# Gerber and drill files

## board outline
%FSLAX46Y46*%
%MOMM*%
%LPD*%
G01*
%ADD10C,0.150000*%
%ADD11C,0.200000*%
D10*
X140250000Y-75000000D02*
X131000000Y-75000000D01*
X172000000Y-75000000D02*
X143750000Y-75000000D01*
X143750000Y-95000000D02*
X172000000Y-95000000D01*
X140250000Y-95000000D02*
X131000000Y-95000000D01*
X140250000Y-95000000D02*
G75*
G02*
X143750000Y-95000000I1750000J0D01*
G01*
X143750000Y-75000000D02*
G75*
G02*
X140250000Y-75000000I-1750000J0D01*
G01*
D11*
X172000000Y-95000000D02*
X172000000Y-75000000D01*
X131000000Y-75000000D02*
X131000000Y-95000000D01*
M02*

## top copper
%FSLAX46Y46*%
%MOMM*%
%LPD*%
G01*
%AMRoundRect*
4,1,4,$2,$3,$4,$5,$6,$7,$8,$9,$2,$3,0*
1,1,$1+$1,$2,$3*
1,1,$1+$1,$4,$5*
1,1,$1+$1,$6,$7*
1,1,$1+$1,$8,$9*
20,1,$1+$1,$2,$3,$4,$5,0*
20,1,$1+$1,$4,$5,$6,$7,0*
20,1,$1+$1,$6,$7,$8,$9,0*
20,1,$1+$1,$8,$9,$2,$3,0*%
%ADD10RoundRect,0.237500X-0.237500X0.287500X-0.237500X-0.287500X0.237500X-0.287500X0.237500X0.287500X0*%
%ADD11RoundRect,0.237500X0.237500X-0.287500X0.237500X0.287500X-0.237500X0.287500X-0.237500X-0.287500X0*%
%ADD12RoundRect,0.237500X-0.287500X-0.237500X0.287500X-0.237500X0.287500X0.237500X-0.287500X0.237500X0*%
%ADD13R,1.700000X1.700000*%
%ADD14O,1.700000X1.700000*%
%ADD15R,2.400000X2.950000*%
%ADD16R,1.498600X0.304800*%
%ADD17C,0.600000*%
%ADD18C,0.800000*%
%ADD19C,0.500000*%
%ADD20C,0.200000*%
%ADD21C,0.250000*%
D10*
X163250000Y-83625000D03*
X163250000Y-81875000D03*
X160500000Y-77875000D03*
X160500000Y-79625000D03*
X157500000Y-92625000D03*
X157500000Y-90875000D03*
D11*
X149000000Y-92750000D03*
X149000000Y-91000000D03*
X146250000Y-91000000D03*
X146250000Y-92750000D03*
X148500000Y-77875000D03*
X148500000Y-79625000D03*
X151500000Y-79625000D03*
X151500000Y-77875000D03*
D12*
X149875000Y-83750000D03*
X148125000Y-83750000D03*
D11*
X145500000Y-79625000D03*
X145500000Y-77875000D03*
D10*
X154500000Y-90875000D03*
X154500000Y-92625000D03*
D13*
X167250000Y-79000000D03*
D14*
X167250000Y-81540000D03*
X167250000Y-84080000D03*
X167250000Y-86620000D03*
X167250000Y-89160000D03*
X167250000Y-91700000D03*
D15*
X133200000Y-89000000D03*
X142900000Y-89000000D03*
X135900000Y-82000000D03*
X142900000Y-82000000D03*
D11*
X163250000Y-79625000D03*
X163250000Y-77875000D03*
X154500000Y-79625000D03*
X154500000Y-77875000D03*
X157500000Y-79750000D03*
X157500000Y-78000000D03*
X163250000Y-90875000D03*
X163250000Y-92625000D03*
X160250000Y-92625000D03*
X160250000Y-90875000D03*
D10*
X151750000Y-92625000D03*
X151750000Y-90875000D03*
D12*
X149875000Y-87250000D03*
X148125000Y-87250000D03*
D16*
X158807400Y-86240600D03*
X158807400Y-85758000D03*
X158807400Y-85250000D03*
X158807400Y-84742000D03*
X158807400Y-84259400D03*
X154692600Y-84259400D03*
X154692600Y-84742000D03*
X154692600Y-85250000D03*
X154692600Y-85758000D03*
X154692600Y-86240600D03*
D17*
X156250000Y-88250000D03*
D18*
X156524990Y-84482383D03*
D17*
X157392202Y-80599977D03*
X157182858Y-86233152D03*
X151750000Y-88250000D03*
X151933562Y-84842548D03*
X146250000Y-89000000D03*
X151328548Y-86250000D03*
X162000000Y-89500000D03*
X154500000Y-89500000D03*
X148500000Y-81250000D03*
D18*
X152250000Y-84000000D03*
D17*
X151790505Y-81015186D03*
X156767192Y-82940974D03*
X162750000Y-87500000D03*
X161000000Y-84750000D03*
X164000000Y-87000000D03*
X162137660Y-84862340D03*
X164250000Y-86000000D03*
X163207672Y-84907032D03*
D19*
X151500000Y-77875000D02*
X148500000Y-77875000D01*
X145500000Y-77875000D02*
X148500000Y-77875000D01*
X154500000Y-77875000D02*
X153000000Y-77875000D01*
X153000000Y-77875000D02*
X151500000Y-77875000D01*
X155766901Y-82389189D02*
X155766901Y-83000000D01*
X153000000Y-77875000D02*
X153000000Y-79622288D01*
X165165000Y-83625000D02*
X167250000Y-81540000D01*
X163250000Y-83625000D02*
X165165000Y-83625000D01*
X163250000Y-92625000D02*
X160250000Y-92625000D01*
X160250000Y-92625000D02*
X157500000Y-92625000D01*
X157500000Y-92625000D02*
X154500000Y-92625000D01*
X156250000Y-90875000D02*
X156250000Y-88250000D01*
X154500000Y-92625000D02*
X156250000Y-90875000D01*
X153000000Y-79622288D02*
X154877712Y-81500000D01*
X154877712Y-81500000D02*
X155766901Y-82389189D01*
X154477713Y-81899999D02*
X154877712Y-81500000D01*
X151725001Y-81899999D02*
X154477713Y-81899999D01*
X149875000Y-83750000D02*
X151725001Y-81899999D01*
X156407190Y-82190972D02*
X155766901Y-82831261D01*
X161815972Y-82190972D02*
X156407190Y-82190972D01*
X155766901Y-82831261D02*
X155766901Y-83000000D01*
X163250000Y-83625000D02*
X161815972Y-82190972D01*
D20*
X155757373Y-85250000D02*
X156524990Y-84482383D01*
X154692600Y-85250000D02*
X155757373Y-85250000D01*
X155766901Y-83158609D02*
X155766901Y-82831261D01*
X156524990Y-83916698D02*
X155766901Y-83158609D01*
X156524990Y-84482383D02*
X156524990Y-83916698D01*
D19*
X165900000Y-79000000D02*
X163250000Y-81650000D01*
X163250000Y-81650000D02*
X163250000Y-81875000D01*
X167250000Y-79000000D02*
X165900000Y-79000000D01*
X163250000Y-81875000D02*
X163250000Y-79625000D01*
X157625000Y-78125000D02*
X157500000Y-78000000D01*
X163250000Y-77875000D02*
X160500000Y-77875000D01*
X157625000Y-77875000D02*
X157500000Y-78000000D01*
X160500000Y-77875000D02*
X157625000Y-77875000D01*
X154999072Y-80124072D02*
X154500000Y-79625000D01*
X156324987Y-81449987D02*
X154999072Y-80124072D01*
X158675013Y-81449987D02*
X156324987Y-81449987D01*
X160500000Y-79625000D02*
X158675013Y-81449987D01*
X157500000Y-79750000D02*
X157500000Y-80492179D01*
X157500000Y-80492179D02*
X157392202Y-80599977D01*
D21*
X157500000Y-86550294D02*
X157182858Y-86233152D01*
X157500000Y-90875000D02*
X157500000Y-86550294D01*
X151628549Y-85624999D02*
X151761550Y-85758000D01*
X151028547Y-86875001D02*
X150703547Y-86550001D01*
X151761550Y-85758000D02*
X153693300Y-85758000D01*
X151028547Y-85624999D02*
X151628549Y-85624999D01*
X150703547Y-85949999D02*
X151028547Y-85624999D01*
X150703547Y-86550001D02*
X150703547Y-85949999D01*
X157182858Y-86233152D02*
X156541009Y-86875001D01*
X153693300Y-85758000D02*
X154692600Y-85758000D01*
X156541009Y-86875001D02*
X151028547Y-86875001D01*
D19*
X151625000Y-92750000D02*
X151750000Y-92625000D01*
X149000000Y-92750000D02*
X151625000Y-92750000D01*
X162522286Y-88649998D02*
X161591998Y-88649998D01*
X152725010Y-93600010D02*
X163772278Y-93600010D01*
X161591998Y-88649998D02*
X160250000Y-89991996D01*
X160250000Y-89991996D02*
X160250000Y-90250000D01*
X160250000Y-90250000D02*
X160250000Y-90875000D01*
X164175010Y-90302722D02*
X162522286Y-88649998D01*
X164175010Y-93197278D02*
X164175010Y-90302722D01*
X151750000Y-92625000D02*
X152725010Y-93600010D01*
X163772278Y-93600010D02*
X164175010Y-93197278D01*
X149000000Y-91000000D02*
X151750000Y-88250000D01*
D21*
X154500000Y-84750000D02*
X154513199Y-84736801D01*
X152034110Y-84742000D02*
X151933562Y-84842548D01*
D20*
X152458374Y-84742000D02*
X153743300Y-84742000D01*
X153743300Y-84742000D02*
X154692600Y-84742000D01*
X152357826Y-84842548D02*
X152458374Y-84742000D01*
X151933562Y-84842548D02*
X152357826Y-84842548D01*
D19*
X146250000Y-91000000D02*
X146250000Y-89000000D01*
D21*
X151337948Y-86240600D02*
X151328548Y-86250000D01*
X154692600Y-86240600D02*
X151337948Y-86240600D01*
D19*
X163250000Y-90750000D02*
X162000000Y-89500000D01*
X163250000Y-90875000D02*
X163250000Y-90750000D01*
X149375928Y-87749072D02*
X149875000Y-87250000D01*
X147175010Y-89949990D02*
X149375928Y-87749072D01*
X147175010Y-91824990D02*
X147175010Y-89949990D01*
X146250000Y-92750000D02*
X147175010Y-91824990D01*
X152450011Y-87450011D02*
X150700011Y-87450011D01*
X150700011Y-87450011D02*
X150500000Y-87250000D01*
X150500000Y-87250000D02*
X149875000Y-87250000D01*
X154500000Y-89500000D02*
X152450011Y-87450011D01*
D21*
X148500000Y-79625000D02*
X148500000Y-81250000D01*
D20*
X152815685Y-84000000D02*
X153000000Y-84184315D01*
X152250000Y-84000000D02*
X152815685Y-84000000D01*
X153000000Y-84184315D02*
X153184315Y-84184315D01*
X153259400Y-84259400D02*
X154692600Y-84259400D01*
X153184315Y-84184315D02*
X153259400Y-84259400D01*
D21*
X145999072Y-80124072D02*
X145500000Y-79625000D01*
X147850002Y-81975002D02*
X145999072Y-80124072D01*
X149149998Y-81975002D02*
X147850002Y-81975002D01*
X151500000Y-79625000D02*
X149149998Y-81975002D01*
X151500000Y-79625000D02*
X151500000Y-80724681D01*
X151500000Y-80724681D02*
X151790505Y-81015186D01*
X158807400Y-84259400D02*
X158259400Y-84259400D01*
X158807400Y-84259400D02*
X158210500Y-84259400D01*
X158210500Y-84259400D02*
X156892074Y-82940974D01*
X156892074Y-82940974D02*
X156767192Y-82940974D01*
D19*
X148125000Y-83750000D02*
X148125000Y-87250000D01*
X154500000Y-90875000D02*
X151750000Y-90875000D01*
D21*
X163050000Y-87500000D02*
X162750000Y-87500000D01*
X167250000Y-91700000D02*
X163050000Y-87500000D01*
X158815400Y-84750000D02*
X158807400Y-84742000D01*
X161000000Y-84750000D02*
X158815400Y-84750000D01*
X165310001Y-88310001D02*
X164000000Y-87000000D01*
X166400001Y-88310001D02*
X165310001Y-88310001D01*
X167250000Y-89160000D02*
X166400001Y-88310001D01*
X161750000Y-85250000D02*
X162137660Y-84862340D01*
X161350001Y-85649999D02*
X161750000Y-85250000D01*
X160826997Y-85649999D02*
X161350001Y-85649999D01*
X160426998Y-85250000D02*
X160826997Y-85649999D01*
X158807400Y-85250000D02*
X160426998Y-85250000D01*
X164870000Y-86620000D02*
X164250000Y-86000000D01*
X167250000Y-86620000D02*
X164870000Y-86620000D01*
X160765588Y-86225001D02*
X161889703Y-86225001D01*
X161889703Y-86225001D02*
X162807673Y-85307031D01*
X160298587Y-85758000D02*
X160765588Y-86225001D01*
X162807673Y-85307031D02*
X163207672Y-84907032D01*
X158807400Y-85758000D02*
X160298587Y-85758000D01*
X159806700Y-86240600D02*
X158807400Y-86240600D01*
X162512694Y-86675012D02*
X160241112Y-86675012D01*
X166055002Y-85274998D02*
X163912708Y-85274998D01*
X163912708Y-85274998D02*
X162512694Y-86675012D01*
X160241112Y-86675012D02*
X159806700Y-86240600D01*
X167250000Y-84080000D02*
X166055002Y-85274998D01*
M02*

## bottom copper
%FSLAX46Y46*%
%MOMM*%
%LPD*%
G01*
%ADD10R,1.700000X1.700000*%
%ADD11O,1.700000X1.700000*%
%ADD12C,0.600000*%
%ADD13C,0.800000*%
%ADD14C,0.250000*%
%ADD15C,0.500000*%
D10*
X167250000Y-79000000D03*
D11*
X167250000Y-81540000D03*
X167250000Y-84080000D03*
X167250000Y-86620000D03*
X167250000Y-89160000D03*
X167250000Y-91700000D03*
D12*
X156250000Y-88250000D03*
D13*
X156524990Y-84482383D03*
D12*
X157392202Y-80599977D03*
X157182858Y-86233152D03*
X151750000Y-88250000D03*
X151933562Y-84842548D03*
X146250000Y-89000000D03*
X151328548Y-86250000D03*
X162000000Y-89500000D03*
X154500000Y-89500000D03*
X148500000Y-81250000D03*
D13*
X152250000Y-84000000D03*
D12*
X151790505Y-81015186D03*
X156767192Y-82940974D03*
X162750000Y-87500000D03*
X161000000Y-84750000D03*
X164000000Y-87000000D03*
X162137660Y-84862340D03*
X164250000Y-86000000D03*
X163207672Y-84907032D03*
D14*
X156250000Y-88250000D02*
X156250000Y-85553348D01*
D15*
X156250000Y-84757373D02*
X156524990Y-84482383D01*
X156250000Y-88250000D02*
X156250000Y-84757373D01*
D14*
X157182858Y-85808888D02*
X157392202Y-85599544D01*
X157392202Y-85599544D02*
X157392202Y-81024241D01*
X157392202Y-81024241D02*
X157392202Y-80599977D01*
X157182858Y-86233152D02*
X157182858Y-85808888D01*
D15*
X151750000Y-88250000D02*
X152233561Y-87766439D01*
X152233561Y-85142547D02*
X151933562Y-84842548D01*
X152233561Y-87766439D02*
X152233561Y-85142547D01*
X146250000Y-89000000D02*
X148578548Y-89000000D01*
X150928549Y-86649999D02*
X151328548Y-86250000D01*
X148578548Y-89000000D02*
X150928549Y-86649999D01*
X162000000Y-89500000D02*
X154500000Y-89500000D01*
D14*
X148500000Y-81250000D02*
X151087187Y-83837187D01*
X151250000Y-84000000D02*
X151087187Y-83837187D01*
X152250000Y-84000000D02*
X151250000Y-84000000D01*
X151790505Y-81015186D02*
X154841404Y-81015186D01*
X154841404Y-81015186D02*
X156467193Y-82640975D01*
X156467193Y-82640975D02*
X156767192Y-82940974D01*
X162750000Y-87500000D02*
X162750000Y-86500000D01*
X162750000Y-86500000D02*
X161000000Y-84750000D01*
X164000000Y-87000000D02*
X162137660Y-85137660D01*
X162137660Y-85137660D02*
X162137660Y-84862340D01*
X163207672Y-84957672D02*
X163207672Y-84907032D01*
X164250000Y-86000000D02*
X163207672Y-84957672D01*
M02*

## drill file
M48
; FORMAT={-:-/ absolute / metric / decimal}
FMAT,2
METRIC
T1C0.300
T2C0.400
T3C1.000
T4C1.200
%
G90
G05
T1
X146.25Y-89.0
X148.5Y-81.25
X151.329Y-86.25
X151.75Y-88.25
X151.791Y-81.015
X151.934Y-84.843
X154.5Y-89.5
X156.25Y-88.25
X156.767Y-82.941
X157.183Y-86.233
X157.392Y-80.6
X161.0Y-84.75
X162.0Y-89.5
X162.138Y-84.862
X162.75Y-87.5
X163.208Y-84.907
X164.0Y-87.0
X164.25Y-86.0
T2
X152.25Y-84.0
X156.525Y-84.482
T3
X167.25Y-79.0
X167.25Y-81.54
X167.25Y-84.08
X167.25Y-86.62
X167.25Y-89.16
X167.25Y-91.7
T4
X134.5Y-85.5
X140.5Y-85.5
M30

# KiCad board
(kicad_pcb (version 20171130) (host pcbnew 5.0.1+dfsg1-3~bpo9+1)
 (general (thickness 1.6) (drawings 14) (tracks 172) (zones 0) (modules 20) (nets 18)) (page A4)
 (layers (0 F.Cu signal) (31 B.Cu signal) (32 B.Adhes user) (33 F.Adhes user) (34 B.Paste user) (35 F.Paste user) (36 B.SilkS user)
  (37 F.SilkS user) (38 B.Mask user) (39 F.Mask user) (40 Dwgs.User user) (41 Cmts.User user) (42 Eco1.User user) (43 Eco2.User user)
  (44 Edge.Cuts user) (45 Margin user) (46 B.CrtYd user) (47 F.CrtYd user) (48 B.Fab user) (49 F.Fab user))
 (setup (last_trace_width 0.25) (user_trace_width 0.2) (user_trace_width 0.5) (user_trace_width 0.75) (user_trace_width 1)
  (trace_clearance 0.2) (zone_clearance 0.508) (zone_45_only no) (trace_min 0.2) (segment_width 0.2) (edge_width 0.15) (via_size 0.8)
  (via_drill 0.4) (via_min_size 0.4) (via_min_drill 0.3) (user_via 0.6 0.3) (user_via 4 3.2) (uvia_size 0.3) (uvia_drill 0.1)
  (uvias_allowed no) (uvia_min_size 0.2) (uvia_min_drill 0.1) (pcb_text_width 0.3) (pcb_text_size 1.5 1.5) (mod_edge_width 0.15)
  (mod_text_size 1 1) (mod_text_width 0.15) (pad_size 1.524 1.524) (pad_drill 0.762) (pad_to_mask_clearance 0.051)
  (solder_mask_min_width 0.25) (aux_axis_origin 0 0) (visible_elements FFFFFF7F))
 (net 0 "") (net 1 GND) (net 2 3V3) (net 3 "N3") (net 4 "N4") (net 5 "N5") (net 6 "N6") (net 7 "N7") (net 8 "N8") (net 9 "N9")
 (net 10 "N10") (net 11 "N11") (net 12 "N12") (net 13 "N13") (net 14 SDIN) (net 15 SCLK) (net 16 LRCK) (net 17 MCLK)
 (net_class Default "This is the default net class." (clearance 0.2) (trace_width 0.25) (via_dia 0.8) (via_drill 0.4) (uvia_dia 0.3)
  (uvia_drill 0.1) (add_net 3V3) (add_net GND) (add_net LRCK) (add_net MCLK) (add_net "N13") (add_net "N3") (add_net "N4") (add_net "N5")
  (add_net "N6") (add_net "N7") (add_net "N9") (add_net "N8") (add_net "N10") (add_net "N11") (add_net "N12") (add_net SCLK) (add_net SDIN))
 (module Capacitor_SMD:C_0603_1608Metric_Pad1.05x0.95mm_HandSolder (layer F.Cu) (at 163.25 82.75 270)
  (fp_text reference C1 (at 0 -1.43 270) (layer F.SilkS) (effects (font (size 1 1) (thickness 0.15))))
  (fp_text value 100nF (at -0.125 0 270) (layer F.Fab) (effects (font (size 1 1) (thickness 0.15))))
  (pad 2 smd roundrect (at 0.875 0 270) (size 1.05 0.95) (layers F.Cu F.Paste F.Mask) (roundrect_rratio 0.25) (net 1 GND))
  (pad 1 smd roundrect (at -0.875 0 270) (size 1.05 0.95) (layers F.Cu F.Paste F.Mask) (roundrect_rratio 0.25) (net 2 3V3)))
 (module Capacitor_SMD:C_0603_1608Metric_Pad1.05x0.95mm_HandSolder (layer F.Cu) (at 160.5 78.75 270)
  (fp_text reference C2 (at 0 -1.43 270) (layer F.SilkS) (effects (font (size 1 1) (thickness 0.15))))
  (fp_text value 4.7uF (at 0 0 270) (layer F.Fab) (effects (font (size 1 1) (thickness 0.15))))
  (pad 1 smd roundrect (at -0.875 0 270) (size 1.05 0.95) (layers F.Cu F.Paste F.Mask) (roundrect_rratio 0.25) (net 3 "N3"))
  (pad 2 smd roundrect (at 0.875 0 270) (size 1.05 0.95) (layers F.Cu F.Paste F.Mask) (roundrect_rratio 0.25) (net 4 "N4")))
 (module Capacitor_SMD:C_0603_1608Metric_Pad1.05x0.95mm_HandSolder (layer F.Cu) (at 157.5 91.75 270)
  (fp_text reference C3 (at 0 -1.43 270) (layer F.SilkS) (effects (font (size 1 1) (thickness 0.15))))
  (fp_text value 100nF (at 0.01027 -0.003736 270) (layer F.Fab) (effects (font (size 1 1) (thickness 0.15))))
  (pad 2 smd roundrect (at 0.875 0 270) (size 1.05 0.95) (layers F.Cu F.Paste F.Mask) (roundrect_rratio 0.25) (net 1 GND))
  (pad 1 smd roundrect (at -0.875 0 270) (size 1.05 0.95) (layers F.Cu F.Paste F.Mask) (roundrect_rratio 0.25) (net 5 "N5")))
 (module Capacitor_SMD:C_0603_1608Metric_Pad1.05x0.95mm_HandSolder (layer F.Cu) (at 149 91.875 90)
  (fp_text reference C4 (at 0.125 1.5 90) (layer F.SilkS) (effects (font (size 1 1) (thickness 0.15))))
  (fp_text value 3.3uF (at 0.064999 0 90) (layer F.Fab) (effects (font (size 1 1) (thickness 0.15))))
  (pad 1 smd roundrect (at -0.875 0 90) (size 1.05 0.95) (layers F.Cu F.Paste F.Mask) (roundrect_rratio 0.25) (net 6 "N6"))
  (pad 2 smd roundrect (at 0.875 0 90) (size 1.05 0.95) (layers F.Cu F.Paste F.Mask) (roundrect_rratio 0.25) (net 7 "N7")))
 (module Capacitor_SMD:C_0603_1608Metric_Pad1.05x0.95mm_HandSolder (layer F.Cu) (at 146.25 91.875 90)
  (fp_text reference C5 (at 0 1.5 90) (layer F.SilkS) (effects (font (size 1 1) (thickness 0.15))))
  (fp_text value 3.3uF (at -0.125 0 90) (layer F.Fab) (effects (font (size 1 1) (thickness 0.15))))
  (pad 2 smd roundrect (at 0.875 0 90) (size 1.05 0.95) (layers F.Cu F.Paste F.Mask) (roundrect_rratio 0.25) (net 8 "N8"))
  (pad 1 smd roundrect (at -0.875 0 90) (size 1.05 0.95) (layers F.Cu F.Paste F.Mask) (roundrect_rratio 0.25) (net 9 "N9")))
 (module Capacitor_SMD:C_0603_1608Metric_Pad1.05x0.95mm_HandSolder (layer F.Cu) (at 148.5 78.75 90)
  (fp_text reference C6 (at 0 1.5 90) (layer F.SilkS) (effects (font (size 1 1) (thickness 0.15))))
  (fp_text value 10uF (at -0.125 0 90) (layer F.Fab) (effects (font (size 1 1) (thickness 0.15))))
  (pad 2 smd roundrect (at 0.875 0 90) (size 1.05 0.95) (layers F.Cu F.Paste F.Mask) (roundrect_rratio 0.25) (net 1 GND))
  (pad 1 smd roundrect (at -0.875 0 90) (size 1.05 0.95) (layers F.Cu F.Paste F.Mask) (roundrect_rratio 0.25) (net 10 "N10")))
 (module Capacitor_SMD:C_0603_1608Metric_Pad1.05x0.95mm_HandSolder (layer F.Cu) (at 151.5 78.75 90)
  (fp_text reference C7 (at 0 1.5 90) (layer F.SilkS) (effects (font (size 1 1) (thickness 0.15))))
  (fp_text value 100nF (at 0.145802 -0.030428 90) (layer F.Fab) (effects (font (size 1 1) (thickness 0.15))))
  (pad 1 smd roundrect (at -0.875 0 90) (size 1.05 0.95) (layers F.Cu F.Paste F.Mask) (roundrect_rratio 0.25) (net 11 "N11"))
  (pad 2 smd roundrect (at 0.875 0 90) (size 1.05 0.95) (layers F.Cu F.Paste F.Mask) (roundrect_rratio 0.25) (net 1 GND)))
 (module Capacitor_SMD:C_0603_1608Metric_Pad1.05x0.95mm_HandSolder (layer F.Cu) (at 149 83.75)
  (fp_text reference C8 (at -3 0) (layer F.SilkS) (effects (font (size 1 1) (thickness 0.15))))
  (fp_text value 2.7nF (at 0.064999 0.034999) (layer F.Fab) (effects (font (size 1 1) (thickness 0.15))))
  (pad 2 smd roundrect (at 0.875 0) (size 1.05 0.95) (layers F.Cu F.Paste F.Mask) (roundrect_rratio 0.25) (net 1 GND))
  (pad 1 smd roundrect (at -0.875 0) (size 1.05 0.95) (layers F.Cu F.Paste F.Mask) (roundrect_rratio 0.25) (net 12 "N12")))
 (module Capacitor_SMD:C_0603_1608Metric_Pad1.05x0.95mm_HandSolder (layer F.Cu) (at 145.5 78.75 90)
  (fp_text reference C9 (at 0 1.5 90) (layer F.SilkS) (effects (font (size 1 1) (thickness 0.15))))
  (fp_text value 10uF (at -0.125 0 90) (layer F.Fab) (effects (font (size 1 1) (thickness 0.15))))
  (pad 1 smd roundrect (at -0.875 0 90) (size 1.05 0.95) (layers F.Cu F.Paste F.Mask) (roundrect_rratio 0.25) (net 11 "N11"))
  (pad 2 smd roundrect (at 0.875 0 90) (size 1.05 0.95) (layers F.Cu F.Paste F.Mask) (roundrect_rratio 0.25) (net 1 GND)))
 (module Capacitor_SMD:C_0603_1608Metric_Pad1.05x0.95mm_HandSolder (layer F.Cu) (at 154.5 91.75 270)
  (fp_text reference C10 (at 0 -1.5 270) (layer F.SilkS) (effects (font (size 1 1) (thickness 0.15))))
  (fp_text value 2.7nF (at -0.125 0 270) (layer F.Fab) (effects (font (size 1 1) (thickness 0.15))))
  (pad 1 smd roundrect (at -0.875 0 270) (size 1.05 0.95) (layers F.Cu F.Paste F.Mask) (roundrect_rratio 0.25) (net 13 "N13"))
  (pad 2 smd roundrect (at 0.875 0 270) (size 1.05 0.95) (layers F.Cu F.Paste F.Mask) (roundrect_rratio 0.25) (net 1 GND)))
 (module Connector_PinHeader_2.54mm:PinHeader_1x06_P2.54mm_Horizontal (layer F.Cu) (at 167.25 79)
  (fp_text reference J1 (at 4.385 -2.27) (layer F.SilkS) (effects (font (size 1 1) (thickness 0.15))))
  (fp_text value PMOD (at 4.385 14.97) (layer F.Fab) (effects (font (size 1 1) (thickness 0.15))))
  (pad 1 thru_hole rect (at 0 0) (size 1.7 1.7) (drill 1) (layers *.Cu *.Mask) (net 2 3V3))
  (pad 2 thru_hole oval (at 0 2.54) (size 1.7 1.7) (drill 1) (layers *.Cu *.Mask) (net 1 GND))
  (pad 3 thru_hole oval (at 0 5.08) (size 1.7 1.7) (drill 1) (layers *.Cu *.Mask) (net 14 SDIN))
  (pad 4 thru_hole oval (at 0 7.62) (size 1.7 1.7) (drill 1) (layers *.Cu *.Mask) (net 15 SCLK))
  (pad 5 thru_hole oval (at 0 10.16) (size 1.7 1.7) (drill 1) (layers *.Cu *.Mask) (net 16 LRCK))
  (pad 6 thru_hole oval (at 0 12.7) (size 1.7 1.7) (drill 1) (layers *.Cu *.Mask) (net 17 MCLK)))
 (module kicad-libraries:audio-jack (layer F.Cu) (at 131.5 85.5)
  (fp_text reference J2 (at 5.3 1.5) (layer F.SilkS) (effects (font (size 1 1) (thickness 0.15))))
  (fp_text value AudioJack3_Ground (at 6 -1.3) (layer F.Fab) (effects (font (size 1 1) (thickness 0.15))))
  (pad 1 smd rect (at 1.7 3.5) (size 2.4 2.95) (layers F.Cu F.Paste F.Mask))
  (pad 2 smd rect (at 11.4 3.5) (size 2.4 2.95) (layers F.Cu F.Paste F.Mask))
  (pad 3 smd rect (at 4.4 -3.5) (size 2.4 2.95) (layers F.Cu F.Paste F.Mask))
  (pad 4 smd rect (at 11.4 -3.5) (size 2.4 2.95) (layers F.Cu F.Paste F.Mask))
  (pad "" np_thru_hole circle (at 3 0) (size 1.2 1.2) (drill 1.2) (layers *.Cu *.Mask))
  (pad "" np_thru_hole circle (at 9 0) (size 1.2 1.2) (drill 1.2) (layers *.Cu *.Mask)))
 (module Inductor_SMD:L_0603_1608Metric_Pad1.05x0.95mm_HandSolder (layer F.Cu) (at 163.25 78.75 90)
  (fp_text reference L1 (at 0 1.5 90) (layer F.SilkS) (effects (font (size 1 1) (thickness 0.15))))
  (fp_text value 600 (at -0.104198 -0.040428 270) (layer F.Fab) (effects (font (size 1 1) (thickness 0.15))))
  (pad 1 smd roundrect (at -0.875 0 90) (size 1.05 0.95) (layers F.Cu F.Paste F.Mask) (roundrect_rratio 0.25) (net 2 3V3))
  (pad 2 smd roundrect (at 0.875 0 90) (size 1.05 0.95) (layers F.Cu F.Paste F.Mask) (roundrect_rratio 0.25) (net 3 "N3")))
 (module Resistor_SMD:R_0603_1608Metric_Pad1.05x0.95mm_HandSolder (layer F.Cu) (at 154.5 78.75 90)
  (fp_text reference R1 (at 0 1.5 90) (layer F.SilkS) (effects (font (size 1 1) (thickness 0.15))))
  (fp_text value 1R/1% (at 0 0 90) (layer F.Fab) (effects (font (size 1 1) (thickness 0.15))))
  (pad 1 smd roundrect (at -0.875 0 90) (size 1.05 0.95) (layers F.Cu F.Paste F.Mask) (roundrect_rratio 0.25) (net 4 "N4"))
  (pad 2 smd roundrect (at 0.875 0 90) (size 1.05 0.95) (layers F.Cu F.Paste F.Mask) (roundrect_rratio 0.25) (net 1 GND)))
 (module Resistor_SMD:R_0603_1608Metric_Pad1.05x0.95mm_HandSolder (layer F.Cu) (at 157.5 78.875 90)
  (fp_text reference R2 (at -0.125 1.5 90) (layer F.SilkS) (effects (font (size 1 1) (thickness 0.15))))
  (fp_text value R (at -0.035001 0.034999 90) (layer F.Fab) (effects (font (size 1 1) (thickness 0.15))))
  (pad 1 smd roundrect (at -0.875 0 90) (size 1.05 0.95) (layers F.Cu F.Paste F.Mask) (roundrect_rratio 0.25) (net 5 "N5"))
  (pad 2 smd roundrect (at 0.875 0 90) (size 1.05 0.95) (layers F.Cu F.Paste F.Mask) (roundrect_rratio 0.25) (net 3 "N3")))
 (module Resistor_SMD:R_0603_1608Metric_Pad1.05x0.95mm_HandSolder (layer F.Cu) (at 163.25 91.75 90)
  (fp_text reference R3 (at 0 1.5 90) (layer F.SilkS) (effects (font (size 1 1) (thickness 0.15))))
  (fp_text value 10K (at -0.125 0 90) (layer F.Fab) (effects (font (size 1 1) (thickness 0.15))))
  (pad 2 smd roundrect (at 0.875 0 90) (size 1.05 0.95) (layers F.Cu F.Paste F.Mask) (roundrect_rratio 0.25) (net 9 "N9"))
  (pad 1 smd roundrect (at -0.875 0 90) (size 1.05 0.95) (layers F.Cu F.Paste F.Mask) (roundrect_rratio 0.25) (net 1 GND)))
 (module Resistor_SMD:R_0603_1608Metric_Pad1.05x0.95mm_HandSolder (layer F.Cu) (at 160.25 91.75 90)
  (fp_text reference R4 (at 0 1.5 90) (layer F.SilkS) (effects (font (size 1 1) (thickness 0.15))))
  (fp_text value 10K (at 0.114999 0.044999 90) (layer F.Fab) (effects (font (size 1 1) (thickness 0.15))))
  (pad 1 smd roundrect (at -0.875 0 90) (size 1.05 0.95) (layers F.Cu F.Paste F.Mask) (roundrect_rratio 0.25) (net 1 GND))
  (pad 2 smd roundrect (at 0.875 0 90) (size 1.05 0.95) (layers F.Cu F.Paste F.Mask) (roundrect_rratio 0.25) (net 6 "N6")))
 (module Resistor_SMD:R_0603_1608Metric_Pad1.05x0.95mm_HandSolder (layer F.Cu) (at 151.75 91.75 270)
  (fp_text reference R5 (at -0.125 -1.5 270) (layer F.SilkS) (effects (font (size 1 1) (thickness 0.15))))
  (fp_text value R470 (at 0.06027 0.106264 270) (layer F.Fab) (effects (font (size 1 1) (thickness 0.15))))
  (pad 2 smd roundrect (at 0.875 0 270) (size 1.05 0.95) (layers F.Cu F.Paste F.Mask) (roundrect_rratio 0.25) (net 6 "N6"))
  (pad 1 smd roundrect (at -0.875 0 270) (size 1.05 0.95) (layers F.Cu F.Paste F.Mask) (roundrect_rratio 0.25) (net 13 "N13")))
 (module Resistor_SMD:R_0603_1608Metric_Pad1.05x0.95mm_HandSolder (layer F.Cu) (at 149 87.25)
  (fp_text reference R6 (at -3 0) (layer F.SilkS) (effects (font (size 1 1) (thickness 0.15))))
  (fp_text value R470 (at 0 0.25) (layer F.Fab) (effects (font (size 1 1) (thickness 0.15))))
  (pad 2 smd roundrect (at 0.875 0) (size 1.05 0.95) (layers F.Cu F.Paste F.Mask) (roundrect_rratio 0.25) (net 9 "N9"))
  (pad 1 smd roundrect (at -0.875 0) (size 1.05 0.95) (layers F.Cu F.Paste F.Mask) (roundrect_rratio 0.25) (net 12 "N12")))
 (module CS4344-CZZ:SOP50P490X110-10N (layer F.Cu) (at 156.75 85.25 180)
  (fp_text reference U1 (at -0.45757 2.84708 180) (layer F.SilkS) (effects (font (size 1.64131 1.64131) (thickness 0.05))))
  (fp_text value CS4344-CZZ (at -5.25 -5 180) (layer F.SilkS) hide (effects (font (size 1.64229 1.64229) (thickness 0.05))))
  (pad 1 smd rect (at -2.0574 -0.9906 180) (size 1.4986 0.3048) (layers F.Cu F.Paste F.Mask) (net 14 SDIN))
  (pad 2 smd rect (at -2.0574 -0.508 180) (size 1.4986 0.3048) (layers F.Cu F.Paste F.Mask) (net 15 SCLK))
  (pad 3 smd rect (at -2.0574 0 180) (size 1.4986 0.3048) (layers F.Cu F.Paste F.Mask) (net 16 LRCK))
  (pad 4 smd rect (at -2.0574 0.508 180) (size 1.4986 0.3048) (layers F.Cu F.Paste F.Mask) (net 17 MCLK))
  (pad 5 smd rect (at -2.0574 0.9906 180) (size 1.4986 0.3048) (layers F.Cu F.Paste F.Mask) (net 11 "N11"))
  (pad 6 smd rect (at 2.0574 0.9906 180) (size 1.4986 0.3048) (layers F.Cu F.Paste F.Mask) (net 10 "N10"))
  (pad 7 smd rect (at 2.0574 0.508 180) (size 1.4986 0.3048) (layers F.Cu F.Paste F.Mask) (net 7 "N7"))
  (pad 8 smd rect (at 2.0574 0 180) (size 1.4986 0.3048) (layers F.Cu F.Paste F.Mask) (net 1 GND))
  (pad 9 smd rect (at 2.0574 -0.508 180) (size 1.4986 0.3048) (layers F.Cu F.Paste F.Mask) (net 5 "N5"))
  (pad 10 smd rect (at 2.0574 -0.9906 180) (size 1.4986 0.3048) (layers F.Cu F.Paste F.Mask) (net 8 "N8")))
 (gr_line (start 140.25 75) (end 131 75) (layer Edge.Cuts) (width 0.15))
 (gr_line (start 172 75) (end 143.75 75) (layer Edge.Cuts) (width 0.15))
 (gr_line (start 143.75 95) (end 172 95) (layer Edge.Cuts) (width 0.15))
 (gr_line (start 140.25 95) (end 131 95) (layer Edge.Cuts) (width 0.15))
 (gr_arc (start 142 95) (end 143.75 95) (angle -180) (layer Edge.Cuts) (width 0.15))
 (gr_arc (start 142 75) (end 140.25 75) (angle -180) (layer Edge.Cuts) (width 0.15))
 (gr_line (start 172 95) (end 172 75) (layer Edge.Cuts) (width 0.2))
 (gr_line (start 131 75) (end 131 95) (layer Edge.Cuts) (width 0.2))
 (segment (start 151.5 77.875) (end 148.5 77.875) (width 0.5) (layer F.Cu) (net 1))
 (segment (start 145.5 77.875) (end 148.5 77.875) (width 0.5) (layer F.Cu) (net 1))
 (segment (start 154.5 77.875) (end 153 77.875) (width 0.5) (layer F.Cu) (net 1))
 (segment (start 153 77.875) (end 151.5 77.875) (width 0.5) (layer F.Cu) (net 1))
 (segment (start 155.766901 82.389189) (end 155.766901 83) (width 0.5) (layer F.Cu) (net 1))
 (segment (start 153 77.875) (end 153 79.622288) (width 0.5) (layer F.Cu) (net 1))
 (segment (start 165.165 83.625) (end 167.25 81.54) (width 0.5) (layer F.Cu) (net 1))
 (segment (start 163.25 83.625) (end 165.165 83.625) (width 0.5) (layer F.Cu) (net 1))
 (via (at 156.25 88.25) (size 0.6) (drill 0.3) (layers F.Cu B.Cu) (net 1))
 (segment (start 163.25 92.625) (end 160.25 92.625) (width 0.5) (layer F.Cu) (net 1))
 (segment (start 160.25 92.625) (end 157.5 92.625) (width 0.5) (layer F.Cu) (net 1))
 (segment (start 157.5 92.625) (end 154.5 92.625) (width 0.5) (layer F.Cu) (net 1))
 (segment (start 156.25 90.875) (end 156.25 88.25) (width 0.5) (layer F.Cu) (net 1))
 (segment (start 154.5 92.625) (end 156.25 90.875) (width 0.5) (layer F.Cu) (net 1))
 (segment (start 153 79.622288) (end 154.877712 81.5) (width 0.5) (layer F.Cu) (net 1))
 (segment (start 154.877712 81.5) (end 155.766901 82.389189) (width 0.5) (layer F.Cu) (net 1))
 (segment (start 154.477713 81.899999) (end 154.877712 81.5) (width 0.5) (layer F.Cu) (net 1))
 (segment (start 151.725001 81.899999) (end 154.477713 81.899999) (width 0.5) (layer F.Cu) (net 1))
 (segment (start 149.875 83.75) (end 151.725001 81.899999) (width 0.5) (layer F.Cu) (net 1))
 (segment (start 156.25 88.25) (end 156.25 85.553348) (width 0.25) (layer B.Cu) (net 1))
 (segment (start 156.25 84.757373) (end 156.52499 84.482383) (width 0.5) (layer B.Cu) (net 1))
 (segment (start 156.25 88.25) (end 156.25 84.757373) (width 0.5) (layer B.Cu) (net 1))
 (via (at 156.52499 84.482383) (size 0.8) (drill 0.4) (layers F.Cu B.Cu) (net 1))
 (segment (start 156.40719 82.190972) (end 155.766901 82.831261) (width 0.5) (layer F.Cu) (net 1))
 (segment (start 161.815972 82.190972) (end 156.40719 82.190972) (width 0.5) (layer F.Cu) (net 1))
 (segment (start 155.766901 82.831261) (end 155.766901 83) (width 0.5) (layer F.Cu) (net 1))
 (segment (start 163.25 83.625) (end 161.815972 82.190972) (width 0.5) (layer F.Cu) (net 1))
 (segment (start 155.757373 85.25) (end 156.52499 84.482383) (width 0.2) (layer F.Cu) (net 1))
 (segment (start 154.6926 85.25) (end 155.757373 85.25) (width 0.2) (layer F.Cu) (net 1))
 (segment (start 155.766901 83.158609) (end 155.766901 82.831261) (width 0.2) (layer F.Cu) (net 1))
 (segment (start 156.52499 83.916698) (end 155.766901 83.158609) (width 0.2) (layer F.Cu) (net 1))
 (segment (start 156.52499 84.482383) (end 156.52499 83.916698) (width 0.2) (layer F.Cu) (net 1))
 (segment (start 165.9 79) (end 163.25 81.65) (width 0.5) (layer F.Cu) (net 2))
 (segment (start 163.25 81.65) (end 163.25 81.875) (width 0.5) (layer F.Cu) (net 2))
 (segment (start 167.25 79) (end 165.9 79) (width 0.5) (layer F.Cu) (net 2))
 (segment (start 163.25 81.875) (end 163.25 79.625) (width 0.5) (layer F.Cu) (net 2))
 (segment (start 157.625 78.125) (end 157.5 78) (width 0.5) (layer F.Cu) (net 3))
 (segment (start 163.25 77.875) (end 160.5 77.875) (width 0.5) (layer F.Cu) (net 3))
 (segment (start 157.625 77.875) (end 157.5 78) (width 0.5) (layer F.Cu) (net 3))
 (segment (start 160.5 77.875) (end 157.625 77.875) (width 0.5) (layer F.Cu) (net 3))
 (segment (start 154.999072 80.124072) (end 154.5 79.625) (width 0.5) (layer F.Cu) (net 4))
 (segment (start 156.324987 81.449987) (end 154.999072 80.124072) (width 0.5) (layer F.Cu) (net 4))
 (segment (start 158.675013 81.449987) (end 156.324987 81.449987) (width 0.5) (layer F.Cu) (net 4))
 (segment (start 160.5 79.625) (end 158.675013 81.449987) (width 0.5) (layer F.Cu) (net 4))
 (via (at 157.392202 80.599977) (size 0.6) (drill 0.3) (layers F.Cu B.Cu) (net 5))
 (segment (start 157.5 79.75) (end 157.5 80.492179) (width 0.5) (layer F.Cu) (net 5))
 (segment (start 157.5 80.492179) (end 157.392202 80.599977) (width 0.5) (layer F.Cu) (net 5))
 (via (at 157.182858 86.233152) (size 0.6) (drill 0.3) (layers F.Cu B.Cu) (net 5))
 (segment (start 157.5 86.550294) (end 157.182858 86.233152) (width 0.25) (layer F.Cu) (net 5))
 (segment (start 157.5 90.875) (end 157.5 86.550294) (width 0.25) (layer F.Cu) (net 5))
 (segment (start 151.628549 85.624999) (end 151.76155 85.758) (width 0.25) (layer F.Cu) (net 5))
 (segment (start 151.028547 86.875001) (end 150.703547 86.550001) (width 0.25) (layer F.Cu) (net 5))
 (segment (start 151.76155 85.758) (end 153.6933 85.758) (width 0.25) (layer F.Cu) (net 5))
 (segment (start 151.028547 85.624999) (end 151.628549 85.624999) (width 0.25) (layer F.Cu) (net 5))
 (segment (start 150.703547 85.949999) (end 151.028547 85.624999) (width 0.25) (layer F.Cu) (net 5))
 (segment (start 150.703547 86.550001) (end 150.703547 85.949999) (width 0.25) (layer F.Cu) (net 5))
 (segment (start 157.182858 86.233152) (end 156.541009 86.875001) (width 0.25) (layer F.Cu) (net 5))
 (segment (start 153.6933 85.758) (end 154.6926 85.758) (width 0.25) (layer F.Cu) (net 5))
 (segment (start 156.541009 86.875001) (end 151.028547 86.875001) (width 0.25) (layer F.Cu) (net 5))
 (segment (start 157.182858 85.808888) (end 157.392202 85.599544) (width 0.25) (layer B.Cu) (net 5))
 (segment (start 157.392202 85.599544) (end 157.392202 81.024241) (width 0.25) (layer B.Cu) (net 5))
 (segment (start 157.392202 81.024241) (end 157.392202 80.599977) (width 0.25) (layer B.Cu) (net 5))
 (segment (start 157.182858 86.233152) (end 157.182858 85.808888) (width 0.25) (layer B.Cu) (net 5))
 (segment (start 151.625 92.75) (end 151.75 92.625) (width 0.5) (layer F.Cu) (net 6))
 (segment (start 149 92.75) (end 151.625 92.75) (width 0.5) (layer F.Cu) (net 6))
 (segment (start 162.522286 88.649998) (end 161.591998 88.649998) (width 0.5) (layer F.Cu) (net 6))
 (segment (start 152.72501 93.60001) (end 163.772278 93.60001) (width 0.5) (layer F.Cu) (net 6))
 (segment (start 161.591998 88.649998) (end 160.25 89.991996) (width 0.5) (layer F.Cu) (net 6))
 (segment (start 160.25 89.991996) (end 160.25 90.25) (width 0.5) (layer F.Cu) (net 6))
 (segment (start 160.25 90.25) (end 160.25 90.875) (width 0.5) (layer F.Cu) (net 6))
 (segment (start 164.17501 90.302722) (end 162.522286 88.649998) (width 0.5) (layer F.Cu) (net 6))
 (segment (start 164.17501 93.197278) (end 164.17501 90.302722) (width 0.5) (layer F.Cu) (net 6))
 (segment (start 151.75 92.625) (end 152.72501 93.60001) (width 0.5) (layer F.Cu) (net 6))
 (segment (start 163.772278 93.60001) (end 164.17501 93.197278) (width 0.5) (layer F.Cu) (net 6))
 (via (at 151.75 88.25) (size 0.6) (drill 0.3) (layers F.Cu B.Cu) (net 7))
 (segment (start 149 91) (end 151.75 88.25) (width 0.5) (layer F.Cu) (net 7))
 (segment (start 154.5 84.75) (end 154.513199 84.736801) (width 0.25) (layer F.Cu) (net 7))
 (via (at 151.933562 84.842548) (size 0.6) (drill 0.3) (layers F.Cu B.Cu) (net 7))
 (segment (start 151.75 88.25) (end 152.233561 87.766439) (width 0.5) (layer B.Cu) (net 7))
 (segment (start 152.03411 84.742) (end 151.933562 84.842548) (width 0.25) (layer F.Cu) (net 7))
 (segment (start 152.233561 85.142547) (end 151.933562 84.842548) (width 0.5) (layer B.Cu) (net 7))
 (segment (start 152.233561 87.766439) (end 152.233561 85.142547) (width 0.5) (layer B.Cu) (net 7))
 (segment (start 152.458374 84.742) (end 153.7433 84.742) (width 0.2) (layer F.Cu) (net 7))
 (segment (start 153.7433 84.742) (end 154.6926 84.742) (width 0.2) (layer F.Cu) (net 7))
 (segment (start 152.357826 84.842548) (end 152.458374 84.742) (width 0.2) (layer F.Cu) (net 7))
 (segment (start 151.933562 84.842548) (end 152.357826 84.842548) (width 0.2) (layer F.Cu) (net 7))
 (via (at 146.25 89) (size 0.6) (drill 0.3) (layers F.Cu B.Cu) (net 8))
 (segment (start 146.25 91) (end 146.25 89) (width 0.5) (layer F.Cu) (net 8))
 (segment (start 146.25 89) (end 148.578548 89) (width 0.5) (layer B.Cu) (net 8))
 (segment (start 150.928549 86.649999) (end 151.328548 86.25) (width 0.5) (layer B.Cu) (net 8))
 (segment (start 151.337948 86.2406) (end 151.328548 86.25) (width 0.25) (layer F.Cu) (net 8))
 (segment (start 154.6926 86.2406) (end 151.337948 86.2406) (width 0.25) (layer F.Cu) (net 8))
 (via (at 151.328548 86.25) (size 0.6) (drill 0.3) (layers F.Cu B.Cu) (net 8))
 (segment (start 148.578548 89) (end 150.928549 86.649999) (width 0.5) (layer B.Cu) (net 8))
 (via (at 162 89.5) (size 0.6) (drill 0.3) (layers F.Cu B.Cu) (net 9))
 (segment (start 163.25 90.75) (end 162 89.5) (width 0.5) (layer F.Cu) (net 9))
 (segment (start 163.25 90.875) (end 163.25 90.75) (width 0.5) (layer F.Cu) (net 9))
 (via (at 154.5 89.5) (size 0.6) (drill 0.3) (layers F.Cu B.Cu) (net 9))
 (segment (start 162 89.5) (end 154.5 89.5) (width 0.5) (layer B.Cu) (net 9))
 (segment (start 149.375928 87.749072) (end 149.875 87.25) (width 0.5) (layer F.Cu) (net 9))
 (segment (start 147.17501 89.94999) (end 149.375928 87.749072) (width 0.5) (layer F.Cu) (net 9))
 (segment (start 147.17501 91.82499) (end 147.17501 89.94999) (width 0.5) (layer F.Cu) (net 9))
 (segment (start 146.25 92.75) (end 147.17501 91.82499) (width 0.5) (layer F.Cu) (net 9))
 (segment (start 152.450011 87.450011) (end 150.700011 87.450011) (width 0.5) (layer F.Cu) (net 9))
 (segment (start 150.700011 87.450011) (end 150.5 87.25) (width 0.5) (layer F.Cu) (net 9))
 (segment (start 150.5 87.25) (end 149.875 87.25) (width 0.5) (layer F.Cu) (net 9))
 (segment (start 154.5 89.5) (end 152.450011 87.450011) (width 0.5) (layer F.Cu) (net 9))
 (via (at 148.5 81.25) (size 0.6) (drill 0.3) (layers F.Cu B.Cu) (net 10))
 (segment (start 148.5 79.625) (end 148.5 81.25) (width 0.25) (layer F.Cu) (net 10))
 (segment (start 148.5 81.25) (end 151.087187 83.837187) (width 0.25) (layer B.Cu) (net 10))
 (via (at 152.25 84) (size 0.8) (drill 0.4) (layers F.Cu B.Cu) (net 10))
 (segment (start 151.25 84) (end 151.087187 83.837187) (width 0.25) (layer B.Cu) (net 10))
 (segment (start 152.25 84) (end 151.25 84) (width 0.25) (layer B.Cu) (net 10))
 (segment (start 152.815685 84) (end 153 84.184315) (width 0.2) (layer F.Cu) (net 10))
 (segment (start 152.25 84) (end 152.815685 84) (width 0.2) (layer F.Cu) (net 10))
 (segment (start 153 84.184315) (end 153.184315 84.184315) (width 0.2) (layer F.Cu) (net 10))
 (segment (start 153.2594 84.2594) (end 154.6926 84.2594) (width 0.2) (layer F.Cu) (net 10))
 (segment (start 153.184315 84.184315) (end 153.2594 84.2594) (width 0.2) (layer F.Cu) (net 10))
 (segment (start 145.999072 80.124072) (end 145.5 79.625) (width 0.25) (layer F.Cu) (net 11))
 (segment (start 147.850002 81.975002) (end 145.999072 80.124072) (width 0.25) (layer F.Cu) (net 11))
 (segment (start 149.149998 81.975002) (end 147.850002 81.975002) (width 0.25) (layer F.Cu) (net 11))
 (segment (start 151.5 79.625) (end 149.149998 81.975002) (width 0.25) (layer F.Cu) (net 11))
 (via (at 151.790505 81.015186) (size 0.6) (drill 0.3) (layers F.Cu B.Cu) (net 11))
 (segment (start 151.5 79.625) (end 151.5 80.724681) (width 0.25) (layer F.Cu) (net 11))
 (segment (start 151.5 80.724681) (end 151.790505 81.015186) (width 0.25) (layer F.Cu) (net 11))
 (segment (start 158.8074 84.2594) (end 158.2594 84.2594) (width 0.25) (layer F.Cu) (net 11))
 (via (at 156.767192 82.940974) (size 0.6) (drill 0.3) (layers F.Cu B.Cu) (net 11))
 (segment (start 151.790505 81.015186) (end 154.841404 81.015186) (width 0.25) (layer B.Cu) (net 11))
 (segment (start 158.8074 84.2594) (end 158.2105 84.2594) (width 0.25) (layer F.Cu) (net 11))
 (segment (start 154.841404 81.015186) (end 156.467193 82.640975) (width 0.25) (layer B.Cu) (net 11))
 (segment (start 158.2105 84.2594) (end 156.892074 82.940974) (width 0.25) (layer F.Cu) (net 11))
 (segment (start 156.892074 82.940974) (end 156.767192 82.940974) (width 0.25) (layer F.Cu) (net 11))
 (segment (start 156.467193 82.640975) (end 156.767192 82.940974) (width 0.25) (layer B.Cu) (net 11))
 (segment (start 148.125 83.75) (end 148.125 87.25) (width 0.5) (layer F.Cu) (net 12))
 (segment (start 154.5 90.875) (end 151.75 90.875) (width 0.5) (layer F.Cu) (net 13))
 (via (at 162.75 87.5) (size 0.6) (drill 0.3) (layers F.Cu B.Cu) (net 17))
 (segment (start 163.05 87.5) (end 162.75 87.5) (width 0.25) (layer F.Cu) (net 17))
 (segment (start 167.25 91.7) (end 163.05 87.5) (width 0.25) (layer F.Cu) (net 17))
 (via (at 161 84.75) (size 0.6) (drill 0.3) (layers F.Cu B.Cu) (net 17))
 (segment (start 162.75 87.5) (end 162.75 86.5) (width 0.25) (layer B.Cu) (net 17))
 (segment (start 162.75 86.5) (end 161 84.75) (width 0.25) (layer B.Cu) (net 17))
 (segment (start 158.8154 84.75) (end 158.8074 84.742) (width 0.25) (layer F.Cu) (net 17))
 (segment (start 161 84.75) (end 158.8154 84.75) (width 0.25) (layer F.Cu) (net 17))
 (via (at 164 87) (size 0.6) (drill 0.3) (layers F.Cu B.Cu) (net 16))
 (segment (start 165.310001 88.310001) (end 164 87) (width 0.25) (layer F.Cu) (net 16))
 (segment (start 166.400001 88.310001) (end 165.310001 88.310001) (width 0.25) (layer F.Cu) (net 16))
 (segment (start 167.25 89.16) (end 166.400001 88.310001) (width 0.25) (layer F.Cu) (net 16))
 (via (at 162.13766 84.86234) (size 0.6) (drill 0.3) (layers F.Cu B.Cu) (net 16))
 (segment (start 164 87) (end 162.13766 85.13766) (width 0.25) (layer B.Cu) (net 16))
 (segment (start 161.75 85.25) (end 162.13766 84.86234) (width 0.25) (layer F.Cu) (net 16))
 (segment (start 161.350001 85.649999) (end 161.75 85.25) (width 0.25) (layer F.Cu) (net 16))
 (segment (start 160.826997 85.649999) (end 161.350001 85.649999) (width 0.25) (layer F.Cu) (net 16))
 (segment (start 160.426998 85.25) (end 160.826997 85.649999) (width 0.25) (layer F.Cu) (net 16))
 (segment (start 158.8074 85.25) (end 160.426998 85.25) (width 0.25) (layer F.Cu) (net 16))
 (segment (start 162.13766 85.13766) (end 162.13766 84.86234) (width 0.25) (layer B.Cu) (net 16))
 (segment (start 164.87 86.62) (end 164.25 86) (width 0.25) (layer F.Cu) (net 15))
 (via (at 164.25 86) (size 0.6) (drill 0.3) (layers F.Cu B.Cu) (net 15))
 (segment (start 167.25 86.62) (end 164.87 86.62) (width 0.25) (layer F.Cu) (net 15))
 (segment (start 160.765588 86.225001) (end 161.889703 86.225001) (width 0.25) (layer F.Cu) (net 15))
 (segment (start 161.889703 86.225001) (end 162.807673 85.307031) (width 0.25) (layer F.Cu) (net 15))
 (segment (start 163.207672 84.957672) (end 163.207672 84.907032) (width 0.25) (layer B.Cu) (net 15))
 (via (at 163.207672 84.907032) (size 0.6) (drill 0.3) (layers F.Cu B.Cu) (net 15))
 (segment (start 160.298587 85.758) (end 160.765588 86.225001) (width 0.25) (layer F.Cu) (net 15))
 (segment (start 164.25 86) (end 163.207672 84.957672) (width 0.25) (layer B.Cu) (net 15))
 (segment (start 162.807673 85.307031) (end 163.207672 84.907032) (width 0.25) (layer F.Cu) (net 15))
 (segment (start 158.8074 85.758) (end 160.298587 85.758) (width 0.25) (layer F.Cu) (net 15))
 (segment (start 159.8067 86.2406) (end 158.8074 86.2406) (width 0.25) (layer F.Cu) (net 14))
 (segment (start 162.512694 86.675012) (end 160.241112 86.675012) (width 0.25) (layer F.Cu) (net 14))
 (segment (start 166.055002 85.274998) (end 163.912708 85.274998) (width 0.25) (layer F.Cu) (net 14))
 (segment (start 163.912708 85.274998) (end 162.512694 86.675012) (width 0.25) (layer F.Cu) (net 14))
 (segment (start 160.241112 86.675012) (end 159.8067 86.2406) (width 0.25) (layer F.Cu) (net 14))
 (segment (start 167.25 84.08) (end 166.055002 85.274998) (width 0.25) (layer F.Cu) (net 14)))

